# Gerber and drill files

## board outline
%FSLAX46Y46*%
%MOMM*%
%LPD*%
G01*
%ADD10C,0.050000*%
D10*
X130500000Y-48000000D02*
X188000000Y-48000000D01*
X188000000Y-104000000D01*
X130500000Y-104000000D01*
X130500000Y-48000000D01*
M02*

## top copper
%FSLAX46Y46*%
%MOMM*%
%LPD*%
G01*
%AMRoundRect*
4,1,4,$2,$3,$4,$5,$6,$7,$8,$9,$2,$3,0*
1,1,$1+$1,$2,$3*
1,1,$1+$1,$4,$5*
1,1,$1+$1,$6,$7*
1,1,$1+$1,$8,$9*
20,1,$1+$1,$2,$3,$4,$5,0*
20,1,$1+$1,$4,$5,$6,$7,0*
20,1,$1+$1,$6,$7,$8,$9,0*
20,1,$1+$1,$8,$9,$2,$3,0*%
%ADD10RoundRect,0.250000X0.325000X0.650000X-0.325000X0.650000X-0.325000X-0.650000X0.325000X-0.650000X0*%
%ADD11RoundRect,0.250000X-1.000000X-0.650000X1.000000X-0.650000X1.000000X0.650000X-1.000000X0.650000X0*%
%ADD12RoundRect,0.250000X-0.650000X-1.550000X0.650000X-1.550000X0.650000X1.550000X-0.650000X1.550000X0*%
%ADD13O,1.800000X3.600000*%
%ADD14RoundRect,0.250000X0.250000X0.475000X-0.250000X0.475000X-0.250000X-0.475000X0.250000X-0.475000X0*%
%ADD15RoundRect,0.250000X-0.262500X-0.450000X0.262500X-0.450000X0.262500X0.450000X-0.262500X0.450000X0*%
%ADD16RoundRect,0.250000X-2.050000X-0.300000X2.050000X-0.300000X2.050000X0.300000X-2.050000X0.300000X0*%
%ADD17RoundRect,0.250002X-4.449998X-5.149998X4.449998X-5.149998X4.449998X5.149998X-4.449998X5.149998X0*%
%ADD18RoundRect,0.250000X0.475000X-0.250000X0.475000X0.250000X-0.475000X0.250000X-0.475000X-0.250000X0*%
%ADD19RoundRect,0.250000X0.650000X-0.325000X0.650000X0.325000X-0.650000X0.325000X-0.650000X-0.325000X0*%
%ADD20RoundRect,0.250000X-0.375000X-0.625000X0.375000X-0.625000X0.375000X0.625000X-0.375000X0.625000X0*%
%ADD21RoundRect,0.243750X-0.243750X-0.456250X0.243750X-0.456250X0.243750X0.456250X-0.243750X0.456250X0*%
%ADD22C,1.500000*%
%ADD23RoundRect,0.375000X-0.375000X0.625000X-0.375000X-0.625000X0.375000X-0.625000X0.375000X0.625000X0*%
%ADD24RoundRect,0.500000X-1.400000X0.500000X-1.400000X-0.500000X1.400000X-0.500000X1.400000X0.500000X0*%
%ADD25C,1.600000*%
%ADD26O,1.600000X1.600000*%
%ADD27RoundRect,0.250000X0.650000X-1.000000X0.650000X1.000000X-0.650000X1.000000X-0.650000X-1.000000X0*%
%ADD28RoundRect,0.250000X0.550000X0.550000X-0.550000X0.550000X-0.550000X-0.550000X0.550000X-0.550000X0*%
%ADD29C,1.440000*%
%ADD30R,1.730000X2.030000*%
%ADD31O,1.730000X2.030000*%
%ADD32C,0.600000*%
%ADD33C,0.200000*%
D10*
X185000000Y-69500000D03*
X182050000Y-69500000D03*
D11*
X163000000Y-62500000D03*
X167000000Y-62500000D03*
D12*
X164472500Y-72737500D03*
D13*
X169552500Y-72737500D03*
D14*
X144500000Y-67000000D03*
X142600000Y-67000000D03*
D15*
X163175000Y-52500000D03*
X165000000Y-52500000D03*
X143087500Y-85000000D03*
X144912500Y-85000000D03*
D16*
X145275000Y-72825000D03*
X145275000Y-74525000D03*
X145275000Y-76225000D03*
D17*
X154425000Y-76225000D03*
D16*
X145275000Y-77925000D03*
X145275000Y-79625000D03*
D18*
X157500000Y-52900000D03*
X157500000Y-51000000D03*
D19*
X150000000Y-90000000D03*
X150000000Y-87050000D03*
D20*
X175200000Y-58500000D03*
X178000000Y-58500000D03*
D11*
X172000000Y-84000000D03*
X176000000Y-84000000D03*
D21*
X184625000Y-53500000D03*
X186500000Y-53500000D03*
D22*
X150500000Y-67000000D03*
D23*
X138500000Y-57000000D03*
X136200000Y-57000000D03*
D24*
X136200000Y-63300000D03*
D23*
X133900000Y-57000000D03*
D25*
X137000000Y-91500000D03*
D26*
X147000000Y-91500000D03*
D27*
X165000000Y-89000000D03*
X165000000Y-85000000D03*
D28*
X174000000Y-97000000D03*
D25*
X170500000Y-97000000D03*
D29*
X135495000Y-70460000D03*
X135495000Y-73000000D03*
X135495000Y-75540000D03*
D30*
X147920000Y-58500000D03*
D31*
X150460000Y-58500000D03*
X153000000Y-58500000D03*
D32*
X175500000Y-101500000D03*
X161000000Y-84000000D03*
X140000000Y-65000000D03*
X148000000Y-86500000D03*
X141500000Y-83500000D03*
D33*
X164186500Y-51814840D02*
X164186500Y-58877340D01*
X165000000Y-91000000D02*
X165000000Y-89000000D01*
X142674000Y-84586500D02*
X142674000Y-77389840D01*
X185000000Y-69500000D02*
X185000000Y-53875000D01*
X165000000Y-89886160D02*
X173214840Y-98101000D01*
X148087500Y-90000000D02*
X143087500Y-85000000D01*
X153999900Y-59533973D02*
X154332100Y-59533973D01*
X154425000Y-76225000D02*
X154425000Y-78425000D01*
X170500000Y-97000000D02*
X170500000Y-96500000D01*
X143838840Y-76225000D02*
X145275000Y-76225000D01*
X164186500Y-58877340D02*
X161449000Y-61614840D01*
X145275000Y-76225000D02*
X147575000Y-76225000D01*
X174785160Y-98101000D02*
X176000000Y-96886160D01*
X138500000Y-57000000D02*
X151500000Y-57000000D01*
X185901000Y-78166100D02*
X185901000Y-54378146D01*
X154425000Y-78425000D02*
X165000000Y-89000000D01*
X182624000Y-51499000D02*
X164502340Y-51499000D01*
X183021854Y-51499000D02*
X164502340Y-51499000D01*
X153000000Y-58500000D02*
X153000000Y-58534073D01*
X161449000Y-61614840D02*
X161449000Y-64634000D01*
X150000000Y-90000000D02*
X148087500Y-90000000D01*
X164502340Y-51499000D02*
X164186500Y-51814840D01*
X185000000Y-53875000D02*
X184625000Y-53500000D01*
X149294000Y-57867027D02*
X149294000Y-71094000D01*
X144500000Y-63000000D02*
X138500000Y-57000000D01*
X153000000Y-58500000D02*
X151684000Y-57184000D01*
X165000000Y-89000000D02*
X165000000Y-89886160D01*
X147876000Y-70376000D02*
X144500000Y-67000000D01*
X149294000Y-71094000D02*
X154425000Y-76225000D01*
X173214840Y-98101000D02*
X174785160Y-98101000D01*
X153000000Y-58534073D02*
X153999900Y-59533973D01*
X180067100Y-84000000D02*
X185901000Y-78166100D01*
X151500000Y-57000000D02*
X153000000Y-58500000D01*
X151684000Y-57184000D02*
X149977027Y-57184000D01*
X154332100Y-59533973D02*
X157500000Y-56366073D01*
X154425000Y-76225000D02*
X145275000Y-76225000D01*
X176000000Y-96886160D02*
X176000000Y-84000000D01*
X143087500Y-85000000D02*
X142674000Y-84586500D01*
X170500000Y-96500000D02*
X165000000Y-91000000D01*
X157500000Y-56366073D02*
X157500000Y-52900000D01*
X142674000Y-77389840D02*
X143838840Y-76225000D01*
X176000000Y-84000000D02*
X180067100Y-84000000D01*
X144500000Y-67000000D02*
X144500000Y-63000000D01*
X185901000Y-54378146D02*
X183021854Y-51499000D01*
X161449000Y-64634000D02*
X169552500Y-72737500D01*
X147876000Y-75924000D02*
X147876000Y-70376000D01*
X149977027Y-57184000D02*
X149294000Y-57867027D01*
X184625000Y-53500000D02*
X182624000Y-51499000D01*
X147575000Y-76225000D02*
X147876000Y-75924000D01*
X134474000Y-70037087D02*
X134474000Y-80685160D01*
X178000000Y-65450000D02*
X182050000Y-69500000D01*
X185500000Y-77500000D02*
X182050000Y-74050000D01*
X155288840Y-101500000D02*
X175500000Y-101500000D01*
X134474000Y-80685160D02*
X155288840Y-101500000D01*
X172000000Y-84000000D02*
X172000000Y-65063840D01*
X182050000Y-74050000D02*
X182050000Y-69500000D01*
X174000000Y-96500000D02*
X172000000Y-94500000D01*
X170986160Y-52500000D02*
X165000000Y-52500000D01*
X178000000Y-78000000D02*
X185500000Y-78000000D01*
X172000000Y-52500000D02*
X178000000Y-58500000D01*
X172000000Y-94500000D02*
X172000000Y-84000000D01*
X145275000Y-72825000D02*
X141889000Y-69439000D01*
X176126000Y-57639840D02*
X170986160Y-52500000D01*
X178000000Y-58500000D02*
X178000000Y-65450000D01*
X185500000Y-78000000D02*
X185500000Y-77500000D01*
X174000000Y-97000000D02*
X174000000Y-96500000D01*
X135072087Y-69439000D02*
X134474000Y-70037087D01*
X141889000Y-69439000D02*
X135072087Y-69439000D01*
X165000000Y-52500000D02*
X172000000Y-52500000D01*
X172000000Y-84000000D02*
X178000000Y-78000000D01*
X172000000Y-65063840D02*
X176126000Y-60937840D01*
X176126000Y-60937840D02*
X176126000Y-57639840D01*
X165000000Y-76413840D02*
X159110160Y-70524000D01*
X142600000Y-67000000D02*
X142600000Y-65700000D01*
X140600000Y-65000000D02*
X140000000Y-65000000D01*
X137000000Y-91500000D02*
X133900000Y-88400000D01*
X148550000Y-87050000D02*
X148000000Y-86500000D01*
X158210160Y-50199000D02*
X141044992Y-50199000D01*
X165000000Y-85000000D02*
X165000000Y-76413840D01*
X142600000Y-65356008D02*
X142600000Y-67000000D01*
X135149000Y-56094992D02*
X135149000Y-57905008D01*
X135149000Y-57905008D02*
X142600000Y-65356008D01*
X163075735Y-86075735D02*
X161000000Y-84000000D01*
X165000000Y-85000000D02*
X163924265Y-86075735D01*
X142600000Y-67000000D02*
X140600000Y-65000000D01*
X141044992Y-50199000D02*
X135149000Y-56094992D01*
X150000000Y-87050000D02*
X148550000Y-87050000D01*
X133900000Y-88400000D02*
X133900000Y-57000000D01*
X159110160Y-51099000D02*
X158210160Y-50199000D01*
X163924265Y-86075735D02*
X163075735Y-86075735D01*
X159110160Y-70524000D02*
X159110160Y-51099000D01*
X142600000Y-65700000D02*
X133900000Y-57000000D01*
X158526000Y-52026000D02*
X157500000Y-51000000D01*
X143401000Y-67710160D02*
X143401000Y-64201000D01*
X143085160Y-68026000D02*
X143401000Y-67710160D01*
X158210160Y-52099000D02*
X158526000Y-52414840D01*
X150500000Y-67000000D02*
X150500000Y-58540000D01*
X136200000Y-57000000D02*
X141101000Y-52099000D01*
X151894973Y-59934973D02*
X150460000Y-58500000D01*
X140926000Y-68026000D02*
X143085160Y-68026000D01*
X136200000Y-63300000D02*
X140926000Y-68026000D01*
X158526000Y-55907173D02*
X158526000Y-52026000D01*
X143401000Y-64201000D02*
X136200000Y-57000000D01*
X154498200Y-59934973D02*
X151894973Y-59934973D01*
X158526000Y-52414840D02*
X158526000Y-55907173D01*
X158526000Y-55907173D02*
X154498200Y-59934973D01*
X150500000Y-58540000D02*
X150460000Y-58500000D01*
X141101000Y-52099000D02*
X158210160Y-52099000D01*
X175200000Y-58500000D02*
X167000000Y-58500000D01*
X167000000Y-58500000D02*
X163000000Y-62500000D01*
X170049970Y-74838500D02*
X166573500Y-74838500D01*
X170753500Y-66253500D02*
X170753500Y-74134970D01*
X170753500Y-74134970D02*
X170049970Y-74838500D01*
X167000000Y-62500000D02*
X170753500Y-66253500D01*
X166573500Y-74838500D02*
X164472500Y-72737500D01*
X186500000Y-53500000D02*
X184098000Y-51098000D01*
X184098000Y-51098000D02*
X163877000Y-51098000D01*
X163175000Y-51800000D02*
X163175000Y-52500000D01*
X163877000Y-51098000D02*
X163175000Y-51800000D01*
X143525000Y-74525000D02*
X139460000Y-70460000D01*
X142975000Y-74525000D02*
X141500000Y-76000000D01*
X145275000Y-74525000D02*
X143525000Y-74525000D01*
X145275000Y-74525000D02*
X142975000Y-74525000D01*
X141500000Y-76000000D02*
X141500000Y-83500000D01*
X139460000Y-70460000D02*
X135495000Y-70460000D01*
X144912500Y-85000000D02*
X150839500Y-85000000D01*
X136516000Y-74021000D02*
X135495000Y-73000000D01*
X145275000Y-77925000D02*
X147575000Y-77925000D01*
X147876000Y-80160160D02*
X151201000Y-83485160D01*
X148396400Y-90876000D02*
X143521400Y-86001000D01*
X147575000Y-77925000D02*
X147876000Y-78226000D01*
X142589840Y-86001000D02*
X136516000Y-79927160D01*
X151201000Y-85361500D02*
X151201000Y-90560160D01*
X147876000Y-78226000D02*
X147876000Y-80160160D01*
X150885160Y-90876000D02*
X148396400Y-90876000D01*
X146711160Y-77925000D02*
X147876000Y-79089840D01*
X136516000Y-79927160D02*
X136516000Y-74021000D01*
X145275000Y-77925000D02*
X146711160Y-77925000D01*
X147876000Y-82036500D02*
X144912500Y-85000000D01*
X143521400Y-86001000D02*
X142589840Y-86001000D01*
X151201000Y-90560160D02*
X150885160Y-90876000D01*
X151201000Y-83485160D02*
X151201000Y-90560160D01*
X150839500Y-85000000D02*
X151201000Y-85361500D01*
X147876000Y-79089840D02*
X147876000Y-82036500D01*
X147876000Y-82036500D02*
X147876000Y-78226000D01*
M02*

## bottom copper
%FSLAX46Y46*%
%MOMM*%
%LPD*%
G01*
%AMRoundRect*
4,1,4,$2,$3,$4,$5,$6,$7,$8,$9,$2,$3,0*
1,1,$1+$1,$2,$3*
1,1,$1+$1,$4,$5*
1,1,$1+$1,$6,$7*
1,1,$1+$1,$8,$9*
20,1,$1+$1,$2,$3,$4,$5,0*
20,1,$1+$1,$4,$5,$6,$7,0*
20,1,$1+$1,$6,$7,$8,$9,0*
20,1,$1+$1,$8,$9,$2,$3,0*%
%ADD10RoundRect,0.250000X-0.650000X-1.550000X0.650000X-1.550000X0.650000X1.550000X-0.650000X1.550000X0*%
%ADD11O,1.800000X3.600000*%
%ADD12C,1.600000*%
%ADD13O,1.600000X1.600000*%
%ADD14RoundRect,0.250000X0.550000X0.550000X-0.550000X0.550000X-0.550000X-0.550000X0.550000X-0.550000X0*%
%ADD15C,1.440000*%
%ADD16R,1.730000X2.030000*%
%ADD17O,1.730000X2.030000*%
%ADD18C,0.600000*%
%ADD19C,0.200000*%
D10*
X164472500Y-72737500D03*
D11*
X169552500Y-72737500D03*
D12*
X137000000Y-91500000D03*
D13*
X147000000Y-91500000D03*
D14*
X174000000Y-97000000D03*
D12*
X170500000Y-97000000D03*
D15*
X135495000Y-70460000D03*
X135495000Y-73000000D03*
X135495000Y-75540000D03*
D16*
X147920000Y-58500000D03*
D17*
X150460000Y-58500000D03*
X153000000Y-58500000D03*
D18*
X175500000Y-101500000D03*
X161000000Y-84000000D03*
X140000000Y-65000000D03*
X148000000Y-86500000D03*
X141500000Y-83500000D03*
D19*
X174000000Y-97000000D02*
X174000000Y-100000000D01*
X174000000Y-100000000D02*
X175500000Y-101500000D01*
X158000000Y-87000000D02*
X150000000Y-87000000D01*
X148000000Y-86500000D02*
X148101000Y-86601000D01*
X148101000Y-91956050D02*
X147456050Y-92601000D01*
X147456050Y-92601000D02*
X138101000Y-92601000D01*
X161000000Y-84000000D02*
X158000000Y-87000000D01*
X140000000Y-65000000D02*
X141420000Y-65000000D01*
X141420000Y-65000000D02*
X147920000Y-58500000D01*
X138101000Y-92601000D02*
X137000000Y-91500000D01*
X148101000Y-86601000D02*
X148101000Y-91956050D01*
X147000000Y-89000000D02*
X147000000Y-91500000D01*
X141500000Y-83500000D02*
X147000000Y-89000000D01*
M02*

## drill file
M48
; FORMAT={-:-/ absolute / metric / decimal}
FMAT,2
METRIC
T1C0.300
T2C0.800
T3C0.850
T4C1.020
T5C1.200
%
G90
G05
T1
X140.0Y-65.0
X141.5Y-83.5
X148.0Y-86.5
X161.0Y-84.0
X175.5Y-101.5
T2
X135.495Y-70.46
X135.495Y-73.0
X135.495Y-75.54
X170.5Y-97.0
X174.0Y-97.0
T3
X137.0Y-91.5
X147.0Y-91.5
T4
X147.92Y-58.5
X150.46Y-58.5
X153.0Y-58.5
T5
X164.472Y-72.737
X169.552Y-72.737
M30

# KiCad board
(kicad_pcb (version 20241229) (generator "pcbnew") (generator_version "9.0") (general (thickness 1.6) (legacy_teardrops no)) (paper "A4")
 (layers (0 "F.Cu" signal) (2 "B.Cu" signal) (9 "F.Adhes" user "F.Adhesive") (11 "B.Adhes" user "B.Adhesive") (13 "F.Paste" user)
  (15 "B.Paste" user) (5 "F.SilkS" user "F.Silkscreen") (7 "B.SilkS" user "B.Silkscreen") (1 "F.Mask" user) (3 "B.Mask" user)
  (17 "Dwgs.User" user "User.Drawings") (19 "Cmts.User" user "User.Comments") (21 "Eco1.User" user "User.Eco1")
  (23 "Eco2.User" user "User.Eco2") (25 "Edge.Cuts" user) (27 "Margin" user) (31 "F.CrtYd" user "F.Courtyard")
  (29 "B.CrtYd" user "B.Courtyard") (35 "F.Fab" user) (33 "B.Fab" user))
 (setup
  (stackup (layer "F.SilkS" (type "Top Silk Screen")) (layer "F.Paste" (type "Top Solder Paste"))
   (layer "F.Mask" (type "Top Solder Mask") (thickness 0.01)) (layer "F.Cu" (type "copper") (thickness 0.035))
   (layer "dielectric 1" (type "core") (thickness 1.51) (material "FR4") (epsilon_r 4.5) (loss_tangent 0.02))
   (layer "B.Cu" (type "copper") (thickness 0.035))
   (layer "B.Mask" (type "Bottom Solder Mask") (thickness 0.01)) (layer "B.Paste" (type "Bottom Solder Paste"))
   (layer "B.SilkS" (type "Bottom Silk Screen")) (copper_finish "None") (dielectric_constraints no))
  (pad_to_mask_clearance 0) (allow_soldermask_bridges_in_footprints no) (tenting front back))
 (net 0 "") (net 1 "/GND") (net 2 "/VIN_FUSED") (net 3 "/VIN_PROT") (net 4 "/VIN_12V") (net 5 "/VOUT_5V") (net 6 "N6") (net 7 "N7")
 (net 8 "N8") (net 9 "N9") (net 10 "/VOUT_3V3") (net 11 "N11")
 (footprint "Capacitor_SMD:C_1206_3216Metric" (layer "F.Cu") (at 183.525 69.5 180)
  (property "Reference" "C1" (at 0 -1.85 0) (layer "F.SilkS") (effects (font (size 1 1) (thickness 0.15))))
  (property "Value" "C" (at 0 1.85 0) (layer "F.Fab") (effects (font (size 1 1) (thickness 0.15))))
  (pad "1" smd roundrect (at -1.475 0 180) (size 1.15 1.8) (layers "F.Cu" "F.Mask" "F.Paste") (roundrect_rratio 0.217391) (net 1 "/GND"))
  (pad "2" smd roundrect (at 1.475 0 180) (size 1.15 1.8) (layers "F.Cu" "F.Mask" "F.Paste") (roundrect_rratio 0.217391)
   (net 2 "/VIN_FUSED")))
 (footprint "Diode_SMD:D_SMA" (layer "F.Cu") (at 165 62.5)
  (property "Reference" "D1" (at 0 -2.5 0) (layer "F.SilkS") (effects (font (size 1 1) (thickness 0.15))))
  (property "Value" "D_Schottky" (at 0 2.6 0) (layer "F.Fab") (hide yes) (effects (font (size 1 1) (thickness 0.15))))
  (pad "1" smd roundrect (at -2 0) (size 2.5 1.8) (layers "F.Cu" "F.Mask" "F.Paste") (roundrect_rratio 0.1388888889) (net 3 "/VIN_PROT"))
  (pad "2" smd roundrect (at 2 0) (size 2.5 1.8) (layers "F.Cu" "F.Mask" "F.Paste") (roundrect_rratio 0.1388888889) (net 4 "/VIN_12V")))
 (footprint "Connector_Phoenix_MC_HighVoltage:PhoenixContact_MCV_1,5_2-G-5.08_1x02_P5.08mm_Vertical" (layer "F.Cu") (at 164.4725 72.7375)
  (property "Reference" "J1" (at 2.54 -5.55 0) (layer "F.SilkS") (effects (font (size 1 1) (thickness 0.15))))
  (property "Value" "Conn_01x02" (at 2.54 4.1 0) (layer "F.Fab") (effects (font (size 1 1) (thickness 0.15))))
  (pad "1" thru_hole roundrect (at 0 0) (size 1.8 3.6) (drill 1.2) (layers "*.Cu" "*.Mask") (remove_unused_layers no)
   (roundrect_rratio 0.138889) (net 4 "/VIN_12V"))
  (pad "2" thru_hole oval (at 5.08 0) (size 1.8 3.6) (drill 1.2) (layers "*.Cu" "*.Mask") (remove_unused_layers no) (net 1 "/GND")))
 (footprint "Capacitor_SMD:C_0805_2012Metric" (layer "F.Cu") (at 143.55 67 180)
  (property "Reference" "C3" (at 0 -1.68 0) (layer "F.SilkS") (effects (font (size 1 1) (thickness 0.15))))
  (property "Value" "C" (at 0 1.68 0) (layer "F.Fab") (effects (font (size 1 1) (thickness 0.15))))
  (pad "1" smd roundrect (at -0.95 0 180) (size 1 1.45) (layers "F.Cu" "F.Mask" "F.Paste") (roundrect_rratio 0.25) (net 1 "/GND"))
  (pad "2" smd roundrect (at 0.95 0 180) (size 1 1.45) (layers "F.Cu" "F.Mask" "F.Paste") (roundrect_rratio 0.25) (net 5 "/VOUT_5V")))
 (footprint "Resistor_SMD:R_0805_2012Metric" (layer "F.Cu") (at 164.0875 52.5)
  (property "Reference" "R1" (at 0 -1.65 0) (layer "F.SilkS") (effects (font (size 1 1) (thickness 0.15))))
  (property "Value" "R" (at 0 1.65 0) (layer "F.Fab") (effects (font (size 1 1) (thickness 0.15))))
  (pad "1" smd roundrect (at -0.9125 0) (size 1.025 1.4) (layers "F.Cu" "F.Mask" "F.Paste") (roundrect_rratio 0.243902) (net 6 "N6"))
  (pad "2" smd roundrect (at 0.9125 0) (size 1.025 1.4) (layers "F.Cu" "F.Mask" "F.Paste") (roundrect_rratio 0.243902) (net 2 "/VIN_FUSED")))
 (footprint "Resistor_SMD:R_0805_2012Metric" (layer "F.Cu") (at 144 85)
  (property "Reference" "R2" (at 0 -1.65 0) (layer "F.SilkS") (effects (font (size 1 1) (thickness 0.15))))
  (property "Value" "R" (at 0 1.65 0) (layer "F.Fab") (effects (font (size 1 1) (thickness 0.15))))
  (pad "1" smd roundrect (at -0.9125 0) (size 1.025 1.4) (layers "F.Cu" "F.Mask" "F.Paste") (roundrect_rratio 0.243902) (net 1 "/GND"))
  (pad "2" smd roundrect (at 0.9125 0) (size 1.025 1.4) (layers "F.Cu" "F.Mask" "F.Paste") (roundrect_rratio 0.243902) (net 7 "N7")))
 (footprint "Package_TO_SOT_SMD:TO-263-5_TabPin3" (layer "F.Cu") (at 152.925 76.225)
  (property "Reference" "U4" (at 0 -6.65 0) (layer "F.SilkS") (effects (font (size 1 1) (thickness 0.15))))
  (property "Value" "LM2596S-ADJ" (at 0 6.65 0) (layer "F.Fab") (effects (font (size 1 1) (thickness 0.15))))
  (pad "" smd roundrect (at -0.925 -2.775) (size 4.55 5.25) (layers "F.Paste") (roundrect_rratio 0.054945))
  (pad "" smd roundrect (at -0.925 2.775) (size 4.55 5.25) (layers "F.Paste") (roundrect_rratio 0.054945))
  (pad "" smd roundrect (at 3.925 -2.775) (size 4.55 5.25) (layers "F.Paste") (roundrect_rratio 0.054945))
  (pad "" smd roundrect (at 3.925 2.775) (size 4.55 5.25) (layers "F.Paste") (roundrect_rratio 0.054945))
  (pad "1" smd roundrect (at -7.65 -3.4) (size 4.6 1.1) (layers "F.Cu" "F.Mask" "F.Paste") (roundrect_rratio 0.227273) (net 2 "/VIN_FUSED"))
  (pad "2" smd roundrect (at -7.65 -1.7) (size 4.6 1.1) (layers "F.Cu" "F.Mask" "F.Paste") (roundrect_rratio 0.227273) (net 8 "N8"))
  (pad "3" smd roundrect (at -7.65 0) (size 4.6 1.1) (layers "F.Cu" "F.Mask" "F.Paste") (roundrect_rratio 0.227273) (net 1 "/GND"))
  (pad "3" smd roundrect (at 1.5 0) (size 9.4 10.8) (layers "F.Cu" "F.Mask") (roundrect_rratio 0.026596) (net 1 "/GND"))
  (pad "4" smd roundrect (at -7.65 1.7) (size 4.6 1.1) (layers "F.Cu" "F.Mask" "F.Paste") (roundrect_rratio 0.227273) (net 7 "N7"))
  (pad "5" smd roundrect (at -7.65 3.4) (size 4.6 1.1) (layers "F.Cu" "F.Mask" "F.Paste") (roundrect_rratio 0.227273) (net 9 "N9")))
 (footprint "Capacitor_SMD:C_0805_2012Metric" (layer "F.Cu") (at 157.5 51.95 90)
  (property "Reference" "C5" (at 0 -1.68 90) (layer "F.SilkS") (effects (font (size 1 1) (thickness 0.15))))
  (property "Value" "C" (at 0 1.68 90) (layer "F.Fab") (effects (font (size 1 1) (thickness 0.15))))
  (pad "1" smd roundrect (at -0.95 0 90) (size 1 1.45) (layers "F.Cu" "F.Mask" "F.Paste") (roundrect_rratio 0.25) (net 1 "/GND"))
  (pad "2" smd roundrect (at 0.95 0 90) (size 1 1.45) (layers "F.Cu" "F.Mask" "F.Paste") (roundrect_rratio 0.25) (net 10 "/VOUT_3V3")))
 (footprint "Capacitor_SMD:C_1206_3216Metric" (layer "F.Cu") (at 150 88.525 90)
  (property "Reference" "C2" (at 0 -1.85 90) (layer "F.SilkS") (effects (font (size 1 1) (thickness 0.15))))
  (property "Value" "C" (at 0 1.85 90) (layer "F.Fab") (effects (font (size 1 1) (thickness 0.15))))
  (pad "1" smd roundrect (at -1.475 0 90) (size 1.15 1.8) (layers "F.Cu" "F.Mask" "F.Paste") (roundrect_rratio 0.217391) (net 1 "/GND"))
  (pad "2" smd roundrect (at 1.475 0 90) (size 1.15 1.8) (layers "F.Cu" "F.Mask" "F.Paste") (roundrect_rratio 0.217391) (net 5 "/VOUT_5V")))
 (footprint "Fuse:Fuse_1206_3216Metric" (layer "F.Cu") (at 176.6 58.5)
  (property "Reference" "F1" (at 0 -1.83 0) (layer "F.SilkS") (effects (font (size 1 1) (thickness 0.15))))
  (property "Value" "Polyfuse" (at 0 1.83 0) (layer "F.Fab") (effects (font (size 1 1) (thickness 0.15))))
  (pad "1" smd roundrect (at -1.4 0) (size 1.25 1.75) (layers "F.Cu" "F.Mask" "F.Paste") (roundrect_rratio 0.2) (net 3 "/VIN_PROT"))
  (pad "2" smd roundrect (at 1.4 0) (size 1.25 1.75) (layers "F.Cu" "F.Mask" "F.Paste") (roundrect_rratio 0.2) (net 2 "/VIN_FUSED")))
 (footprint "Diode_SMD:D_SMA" (layer "F.Cu") (at 174 84)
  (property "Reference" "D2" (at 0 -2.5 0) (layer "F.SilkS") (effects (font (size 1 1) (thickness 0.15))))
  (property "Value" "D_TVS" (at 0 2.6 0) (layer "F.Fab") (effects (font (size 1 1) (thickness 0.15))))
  (pad "1" smd roundrect (at -2 0) (size 2.5 1.8) (layers "F.Cu" "F.Mask" "F.Paste") (roundrect_rratio 0.1388888889) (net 2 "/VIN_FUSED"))
  (pad "2" smd roundrect (at 2 0) (size 2.5 1.8) (layers "F.Cu" "F.Mask" "F.Paste") (roundrect_rratio 0.1388888889) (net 1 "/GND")))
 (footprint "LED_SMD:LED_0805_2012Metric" (layer "F.Cu") (at 185.5625 53.5)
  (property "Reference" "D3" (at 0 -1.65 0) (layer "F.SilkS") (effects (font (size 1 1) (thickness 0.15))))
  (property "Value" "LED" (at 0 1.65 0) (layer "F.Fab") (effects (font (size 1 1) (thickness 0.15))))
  (pad "1" smd roundrect (at -0.9375 0) (size 0.975 1.4) (layers "F.Cu" "F.Mask" "F.Paste") (roundrect_rratio 0.25) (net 1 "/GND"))
  (pad "2" smd roundrect (at 0.9375 0) (size 0.975 1.4) (layers "F.Cu" "F.Mask" "F.Paste") (roundrect_rratio 0.25) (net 6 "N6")))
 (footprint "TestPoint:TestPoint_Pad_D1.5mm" (layer "F.Cu") (at 150.5 67)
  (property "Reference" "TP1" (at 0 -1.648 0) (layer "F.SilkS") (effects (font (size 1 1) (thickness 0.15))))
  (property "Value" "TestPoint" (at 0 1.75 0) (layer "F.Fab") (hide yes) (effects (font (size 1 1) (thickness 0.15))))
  (pad "1" smd circle (at 0 0) (size 1.5 1.5) (layers "F.Cu" "F.Mask") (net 10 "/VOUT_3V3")))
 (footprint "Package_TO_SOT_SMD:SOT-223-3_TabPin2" (layer "F.Cu") (at 136.2 60.15 -90)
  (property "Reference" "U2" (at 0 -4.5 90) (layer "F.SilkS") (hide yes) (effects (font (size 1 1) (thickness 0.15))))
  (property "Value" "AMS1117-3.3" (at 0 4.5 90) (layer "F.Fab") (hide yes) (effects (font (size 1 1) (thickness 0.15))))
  (pad "1" smd roundrect (at -3.15 -2.3 270) (size 2 1.5) (layers "F.Cu" "F.Mask" "F.Paste") (roundrect_rratio 0.25) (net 1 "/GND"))
  (pad "2" smd roundrect (at -3.15 0 270) (size 2 1.5) (layers "F.Cu" "F.Mask" "F.Paste") (roundrect_rratio 0.25) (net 10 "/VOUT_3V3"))
  (pad "2" smd roundrect (at 3.15 0 270) (size 2 3.8) (layers "F.Cu" "F.Mask" "F.Paste") (roundrect_rratio 0.25) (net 10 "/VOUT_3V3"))
  (pad "3" smd roundrect (at -3.15 2.3 270) (size 2 1.5) (layers "F.Cu" "F.Mask" "F.Paste") (roundrect_rratio 0.25) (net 5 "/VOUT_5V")))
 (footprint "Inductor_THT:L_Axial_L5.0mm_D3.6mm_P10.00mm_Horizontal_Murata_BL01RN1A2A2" (layer "F.Cu") (at 137 91.5)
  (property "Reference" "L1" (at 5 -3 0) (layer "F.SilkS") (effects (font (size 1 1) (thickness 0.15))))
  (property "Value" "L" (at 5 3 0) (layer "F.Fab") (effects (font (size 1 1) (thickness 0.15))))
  (pad "1" thru_hole circle (at 0 0) (size 1.6 1.6) (drill 0.85) (layers "*.Cu" "*.Mask") (remove_unused_layers no) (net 5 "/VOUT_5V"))
  (pad "2" thru_hole oval (at 10 0) (size 1.6 1.6) (drill 0.85) (layers "*.Cu" "*.Mask") (remove_unused_layers no) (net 8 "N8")))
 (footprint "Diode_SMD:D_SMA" (layer "F.Cu") (at 165 87 90)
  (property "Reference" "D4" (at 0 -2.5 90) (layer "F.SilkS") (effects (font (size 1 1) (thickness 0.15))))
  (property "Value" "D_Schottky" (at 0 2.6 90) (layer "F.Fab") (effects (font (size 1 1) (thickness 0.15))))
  (pad "1" smd roundrect (at -2 0 90) (size 2.5 1.8) (layers "F.Cu" "F.Mask" "F.Paste") (roundrect_rratio 0.1388888889) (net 1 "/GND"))
  (pad "2" smd roundrect (at 2 0 90) (size 2.5 1.8) (layers "F.Cu" "F.Mask" "F.Paste") (roundrect_rratio 0.1388888889) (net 5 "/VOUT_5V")))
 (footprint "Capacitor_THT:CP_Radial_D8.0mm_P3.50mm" (layer "F.Cu") (at 174 97 180)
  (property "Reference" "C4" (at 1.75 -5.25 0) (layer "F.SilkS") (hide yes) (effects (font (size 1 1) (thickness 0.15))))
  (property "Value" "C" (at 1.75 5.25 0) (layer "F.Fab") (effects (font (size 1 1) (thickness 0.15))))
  (pad "1" thru_hole roundrect (at 0 0 180) (size 1.6 1.6) (drill 0.8) (layers "*.Cu" "*.Mask") (remove_unused_layers no)
   (roundrect_rratio 0.15625) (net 2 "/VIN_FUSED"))
  (pad "2" thru_hole circle (at 3.5 0 180) (size 1.6 1.6) (drill 0.8) (layers "*.Cu" "*.Mask") (remove_unused_layers no) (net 1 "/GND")))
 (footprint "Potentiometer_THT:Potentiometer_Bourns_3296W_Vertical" (layer "F.Cu") (at 135.495 70.46 90)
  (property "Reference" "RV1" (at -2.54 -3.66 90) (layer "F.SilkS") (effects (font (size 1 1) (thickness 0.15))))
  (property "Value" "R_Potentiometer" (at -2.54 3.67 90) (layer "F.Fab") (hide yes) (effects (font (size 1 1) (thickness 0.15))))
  (pad "1" thru_hole circle (at 0 0 90) (size 1.44 1.44) (drill 0.8) (layers "*.Cu" "*.Mask") (remove_unused_layers no) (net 8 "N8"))
  (pad "2" thru_hole circle (at -2.54 0 90) (size 1.44 1.44) (drill 0.8) (layers "*.Cu" "*.Mask") (remove_unused_layers no) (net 7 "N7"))
  (pad "3" thru_hole circle (at -5.08 0 90) (size 1.44 1.44) (drill 0.8) (layers "*.Cu" "*.Mask") (remove_unused_layers no) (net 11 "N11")))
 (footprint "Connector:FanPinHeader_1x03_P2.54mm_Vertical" (layer "F.Cu") (at 147.92 58.5)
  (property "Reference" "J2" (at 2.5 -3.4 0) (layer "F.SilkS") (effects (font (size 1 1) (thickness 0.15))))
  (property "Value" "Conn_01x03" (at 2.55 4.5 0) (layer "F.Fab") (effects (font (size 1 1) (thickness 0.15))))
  (pad "1" thru_hole rect (at 0 0 90) (size 2.03 1.73) (drill 1.02) (layers "*.Cu" "*.Mask") (remove_unused_layers no) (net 5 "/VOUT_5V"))
  (pad "2" thru_hole oval (at 2.54 0 90) (size 2.03 1.73) (drill 1.02) (layers "*.Cu" "*.Mask") (remove_unused_layers no)
   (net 10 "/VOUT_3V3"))
  (pad "3" thru_hole oval (at 5.08 0 90) (size 2.03 1.73) (drill 1.02) (layers "*.Cu" "*.Mask") (remove_unused_layers no) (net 1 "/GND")))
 (gr_rect (start 130.5 48) (end 188 104) (stroke (width 0.05) (type default)) (fill no) (layer "Edge.Cuts"))
 (segment (start 164.1865 51.81484) (end 164.1865 58.87734) (width 0.2) (layer "F.Cu") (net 1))
 (segment (start 165 91) (end 165 89) (width 0.2) (layer "F.Cu") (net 1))
 (segment (start 142.674 84.5865) (end 142.674 77.38984) (width 0.2) (layer "F.Cu") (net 1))
 (segment (start 185 69.5) (end 185 53.875) (width 0.2) (layer "F.Cu") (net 1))
 (segment (start 165 89.88616) (end 173.21484 98.101) (width 0.2) (layer "F.Cu") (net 1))
 (segment (start 148.0875 90) (end 143.0875 85) (width 0.2) (layer "F.Cu") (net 1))
 (segment (start 153.9999 59.533973) (end 154.3321 59.533973) (width 0.2) (layer "F.Cu") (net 1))
 (segment (start 154.425 76.225) (end 154.425 78.425) (width 0.2) (layer "F.Cu") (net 1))
 (segment (start 170.5 97) (end 170.5 96.5) (width 0.2) (layer "F.Cu") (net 1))
 (segment (start 143.83884 76.225) (end 145.275 76.225) (width 0.2) (layer "F.Cu") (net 1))
 (segment (start 164.1865 58.87734) (end 161.449 61.61484) (width 0.2) (layer "F.Cu") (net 1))
 (segment (start 145.275 76.225) (end 147.575 76.225) (width 0.2) (layer "F.Cu") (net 1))
 (segment (start 174.78516 98.101) (end 176 96.88616) (width 0.2) (layer "F.Cu") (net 1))
 (segment (start 138.5 57) (end 151.5 57) (width 0.2) (layer "F.Cu") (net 1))
 (segment (start 185.901 78.1661) (end 185.901 54.378146) (width 0.2) (layer "F.Cu") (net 1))
 (segment (start 154.425 78.425) (end 165 89) (width 0.2) (layer "F.Cu") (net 1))
 (segment (start 182.624 51.499) (end 164.50234 51.499) (width 0.2) (layer "F.Cu") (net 1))
 (segment (start 183.021854 51.499) (end 164.50234 51.499) (width 0.2) (layer "F.Cu") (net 1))
 (segment (start 153 58.5) (end 153 58.534073) (width 0.2) (layer "F.Cu") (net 1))
 (segment (start 161.449 61.61484) (end 161.449 64.634) (width 0.2) (layer "F.Cu") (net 1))
 (segment (start 150 90) (end 148.0875 90) (width 0.2) (layer "F.Cu") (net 1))
 (segment (start 164.50234 51.499) (end 164.1865 51.81484) (width 0.2) (layer "F.Cu") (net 1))
 (segment (start 185 53.875) (end 184.625 53.5) (width 0.2) (layer "F.Cu") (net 1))
 (segment (start 149.294 57.867027) (end 149.294 71.094) (width 0.2) (layer "F.Cu") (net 1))
 (segment (start 144.5 63) (end 138.5 57) (width 0.2) (layer "F.Cu") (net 1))
 (segment (start 153 58.5) (end 151.684 57.184) (width 0.2) (layer "F.Cu") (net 1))
 (segment (start 165 89) (end 165 89.88616) (width 0.2) (layer "F.Cu") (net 1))
 (segment (start 147.876 70.376) (end 144.5 67) (width 0.2) (layer "F.Cu") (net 1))
 (segment (start 149.294 71.094) (end 154.425 76.225) (width 0.2) (layer "F.Cu") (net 1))
 (segment (start 173.21484 98.101) (end 174.78516 98.101) (width 0.2) (layer "F.Cu") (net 1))
 (segment (start 153 58.534073) (end 153.9999 59.533973) (width 0.2) (layer "F.Cu") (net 1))
 (segment (start 180.0671 84) (end 185.901 78.1661) (width 0.2) (layer "F.Cu") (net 1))
 (segment (start 151.5 57) (end 153 58.5) (width 0.2) (layer "F.Cu") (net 1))
 (segment (start 151.684 57.184) (end 149.977027 57.184) (width 0.2) (layer "F.Cu") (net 1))
 (segment (start 154.3321 59.533973) (end 157.5 56.366073) (width 0.2) (layer "F.Cu") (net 1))
 (segment (start 154.425 76.225) (end 145.275 76.225) (width 0.2) (layer "F.Cu") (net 1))
 (segment (start 176 96.88616) (end 176 84) (width 0.2) (layer "F.Cu") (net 1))
 (segment (start 143.0875 85) (end 142.674 84.5865) (width 0.2) (layer "F.Cu") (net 1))
 (segment (start 170.5 96.5) (end 165 91) (width 0.2) (layer "F.Cu") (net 1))
 (segment (start 157.5 56.366073) (end 157.5 52.9) (width 0.2) (layer "F.Cu") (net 1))
 (segment (start 142.674 77.38984) (end 143.83884 76.225) (width 0.2) (layer "F.Cu") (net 1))
 (segment (start 176 84) (end 180.0671 84) (width 0.2) (layer "F.Cu") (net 1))
 (segment (start 144.5 67) (end 144.5 63) (width 0.2) (layer "F.Cu") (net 1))
 (segment (start 185.901 54.378146) (end 183.021854 51.499) (width 0.2) (layer "F.Cu") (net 1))
 (segment (start 161.449 64.634) (end 169.5525 72.7375) (width 0.2) (layer "F.Cu") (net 1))
 (segment (start 147.876 75.924) (end 147.876 70.376) (width 0.2) (layer "F.Cu") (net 1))
 (segment (start 149.977027 57.184) (end 149.294 57.867027) (width 0.2) (layer "F.Cu") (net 1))
 (segment (start 184.625 53.5) (end 182.624 51.499) (width 0.2) (layer "F.Cu") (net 1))
 (segment (start 147.575 76.225) (end 147.876 75.924) (width 0.2) (layer "F.Cu") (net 1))
 (segment (start 134.474 70.037087) (end 134.474 80.68516) (width 0.2) (layer "F.Cu") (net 2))
 (segment (start 178 65.45) (end 182.05 69.5) (width 0.2) (layer "F.Cu") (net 2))
 (segment (start 185.5 77.5) (end 182.05 74.05) (width 0.2) (layer "F.Cu") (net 2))
 (segment (start 155.28884 101.5) (end 175.5 101.5) (width 0.2) (layer "F.Cu") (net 2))
 (segment (start 134.474 80.68516) (end 155.28884 101.5) (width 0.2) (layer "F.Cu") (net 2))
 (segment (start 172 84) (end 172 65.06384) (width 0.2) (layer "F.Cu") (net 2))
 (segment (start 182.05 74.05) (end 182.05 69.5) (width 0.2) (layer "F.Cu") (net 2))
 (segment (start 174 96.5) (end 172 94.5) (width 0.2) (layer "F.Cu") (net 2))
 (segment (start 170.98616 52.5) (end 165 52.5) (width 0.2) (layer "F.Cu") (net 2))
 (segment (start 178 78) (end 185.5 78) (width 0.2) (layer "F.Cu") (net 2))
 (segment (start 172 52.5) (end 178 58.5) (width 0.2) (layer "F.Cu") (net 2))
 (segment (start 172 94.5) (end 172 84) (width 0.2) (layer "F.Cu") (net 2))
 (segment (start 145.275 72.825) (end 141.889 69.439) (width 0.2) (layer "F.Cu") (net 2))
 (segment (start 176.126 57.63984) (end 170.98616 52.5) (width 0.2) (layer "F.Cu") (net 2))
 (segment (start 178 58.5) (end 178 65.45) (width 0.2) (layer "F.Cu") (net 2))
 (segment (start 185.5 78) (end 185.5 77.5) (width 0.2) (layer "F.Cu") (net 2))
 (segment (start 174 97) (end 174 96.5) (width 0.2) (layer "F.Cu") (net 2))
 (segment (start 135.072087 69.439) (end 134.474 70.037087) (width 0.2) (layer "F.Cu") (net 2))
 (segment (start 141.889 69.439) (end 135.072087 69.439) (width 0.2) (layer "F.Cu") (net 2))
 (segment (start 165 52.5) (end 172 52.5) (width 0.2) (layer "F.Cu") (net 2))
 (segment (start 172 84) (end 178 78) (width 0.2) (layer "F.Cu") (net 2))
 (segment (start 172 65.06384) (end 176.126 60.93784) (width 0.2) (layer "F.Cu") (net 2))
 (segment (start 176.126 60.93784) (end 176.126 57.63984) (width 0.2) (layer "F.Cu") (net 2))
 (via (at 175.5 101.5) (size 0.6) (drill 0.3) (layers "F.Cu" "B.Cu") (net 2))
 (segment (start 174 97) (end 174 100) (width 0.2) (layer "B.Cu") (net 2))
 (segment (start 174 100) (end 175.5 101.5) (width 0.2) (layer "B.Cu") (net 2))
 (segment (start 165 76.41384) (end 159.11016 70.524) (width 0.2) (layer "F.Cu") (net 5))
 (segment (start 142.6 67) (end 142.6 65.7) (width 0.2) (layer "F.Cu") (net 5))
 (segment (start 140.6 65) (end 140 65) (width 0.2) (layer "F.Cu") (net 5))
 (segment (start 137 91.5) (end 133.9 88.4) (width 0.2) (layer "F.Cu") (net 5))
 (segment (start 148.55 87.05) (end 148 86.5) (width 0.2) (layer "F.Cu") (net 5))
 (segment (start 158.21016 50.199) (end 141.044992 50.199) (width 0.2) (layer "F.Cu") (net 5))
 (segment (start 165 85) (end 165 76.41384) (width 0.2) (layer "F.Cu") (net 5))
 (segment (start 142.6 65.356008) (end 142.6 67) (width 0.2) (layer "F.Cu") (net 5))
 (segment (start 135.149 56.094992) (end 135.149 57.905008) (width 0.2) (layer "F.Cu") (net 5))
 (segment (start 135.149 57.905008) (end 142.6 65.356008) (width 0.2) (layer "F.Cu") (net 5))
 (segment (start 163.075735 86.075735) (end 161 84) (width 0.2) (layer "F.Cu") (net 5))
 (segment (start 165 85) (end 163.924265 86.075735) (width 0.2) (layer "F.Cu") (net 5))
 (segment (start 142.6 67) (end 140.6 65) (width 0.2) (layer "F.Cu") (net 5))
 (segment (start 141.044992 50.199) (end 135.149 56.094992) (width 0.2) (layer "F.Cu") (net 5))
 (segment (start 150 87.05) (end 148.55 87.05) (width 0.2) (layer "F.Cu") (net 5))
 (segment (start 133.9 88.4) (end 133.9 57) (width 0.2) (layer "F.Cu") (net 5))
 (segment (start 159.11016 51.099) (end 158.21016 50.199) (width 0.2) (layer "F.Cu") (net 5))
 (segment (start 163.924265 86.075735) (end 163.075735 86.075735) (width 0.2) (layer "F.Cu") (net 5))
 (segment (start 159.11016 70.524) (end 159.11016 51.099) (width 0.2) (layer "F.Cu") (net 5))
 (segment (start 142.6 65.7) (end 133.9 57) (width 0.2) (layer "F.Cu") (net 5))
 (via (at 161 84) (size 0.6) (drill 0.3) (layers "F.Cu" "B.Cu") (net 5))
 (via (at 140 65) (size 0.6) (drill 0.3) (layers "F.Cu" "B.Cu") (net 5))
 (via (at 148 86.5) (size 0.6) (drill 0.3) (layers "F.Cu" "B.Cu") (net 5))
 (segment (start 158 87) (end 150 87) (width 0.2) (layer "B.Cu") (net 5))
 (segment (start 148 86.5) (end 148.101 86.601) (width 0.2) (layer "B.Cu") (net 5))
 (segment (start 148.101 91.95605) (end 147.45605 92.601) (width 0.2) (layer "B.Cu") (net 5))
 (segment (start 147.45605 92.601) (end 138.101 92.601) (width 0.2) (layer "B.Cu") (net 5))
 (segment (start 161 84) (end 158 87) (width 0.2) (layer "B.Cu") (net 5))
 (segment (start 140 65) (end 141.42 65) (width 0.2) (layer "B.Cu") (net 5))
 (segment (start 141.42 65) (end 147.92 58.5) (width 0.2) (layer "B.Cu") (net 5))
 (segment (start 138.101 92.601) (end 137 91.5) (width 0.2) (layer "B.Cu") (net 5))
 (segment (start 148.101 86.601) (end 148.101 91.95605) (width 0.2) (layer "B.Cu") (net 5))
 (segment (start 158.526 52.026) (end 157.5 51) (width 0.2) (layer "F.Cu") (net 10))
 (segment (start 143.401 67.71016) (end 143.401 64.201) (width 0.2) (layer "F.Cu") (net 10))
 (segment (start 143.08516 68.026) (end 143.401 67.71016) (width 0.2) (layer "F.Cu") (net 10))
 (segment (start 158.21016 52.099) (end 158.526 52.41484) (width 0.2) (layer "F.Cu") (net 10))
 (segment (start 150.5 67) (end 150.5 58.54) (width 0.2) (layer "F.Cu") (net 10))
 (segment (start 136.2 57) (end 141.101 52.099) (width 0.2) (layer "F.Cu") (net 10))
 (segment (start 151.894973 59.934973) (end 150.46 58.5) (width 0.2) (layer "F.Cu") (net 10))
 (segment (start 140.926 68.026) (end 143.08516 68.026) (width 0.2) (layer "F.Cu") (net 10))
 (segment (start 136.2 63.3) (end 140.926 68.026) (width 0.2) (layer "F.Cu") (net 10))
 (segment (start 158.526 55.907173) (end 158.526 52.026) (width 0.2) (layer "F.Cu") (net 10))
 (segment (start 143.401 64.201) (end 136.2 57) (width 0.2) (layer "F.Cu") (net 10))
 (segment (start 154.4982 59.934973) (end 151.894973 59.934973) (width 0.2) (layer "F.Cu") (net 10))
 (segment (start 158.526 52.41484) (end 158.526 55.907173) (width 0.2) (layer "F.Cu") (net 10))
 (segment (start 158.526 55.907173) (end 154.4982 59.934973) (width 0.2) (layer "F.Cu") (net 10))
 (segment (start 150.5 58.54) (end 150.46 58.5) (width 0.2) (layer "F.Cu") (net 10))
 (segment (start 141.101 52.099) (end 158.21016 52.099) (width 0.2) (layer "F.Cu") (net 10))
 (segment (start 175.2 58.5) (end 167 58.5) (width 0.2) (layer "F.Cu") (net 3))
 (segment (start 167 58.5) (end 163 62.5) (width 0.2) (layer "F.Cu") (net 3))
 (segment (start 170.04997 74.8385) (end 166.5735 74.8385) (width 0.2) (layer "F.Cu") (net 4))
 (segment (start 170.7535 66.2535) (end 170.7535 74.13497) (width 0.2) (layer "F.Cu") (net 4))
 (segment (start 170.7535 74.13497) (end 170.04997 74.8385) (width 0.2) (layer "F.Cu") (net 4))
 (segment (start 167 62.5) (end 170.7535 66.2535) (width 0.2) (layer "F.Cu") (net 4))
 (segment (start 166.5735 74.8385) (end 164.4725 72.7375) (width 0.2) (layer "F.Cu") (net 4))
 (segment (start 186.5 53.5) (end 184.098 51.098) (width 0.2) (layer "F.Cu") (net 6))
 (segment (start 184.098 51.098) (end 163.877 51.098) (width 0.2) (layer "F.Cu") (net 6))
 (segment (start 163.175 51.8) (end 163.175 52.5) (width 0.2) (layer "F.Cu") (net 6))
 (segment (start 163.877 51.098) (end 163.175 51.8) (width 0.2) (layer "F.Cu") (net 6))
 (segment (start 143.525 74.525) (end 139.46 70.46) (width 0.2) (layer "F.Cu") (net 8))
 (segment (start 142.975 74.525) (end 141.5 76) (width 0.2) (layer "F.Cu") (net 8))
 (segment (start 145.275 74.525) (end 143.525 74.525) (width 0.2) (layer "F.Cu") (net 8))
 (segment (start 145.275 74.525) (end 142.975 74.525) (width 0.2) (layer "F.Cu") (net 8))
 (segment (start 141.5 76) (end 141.5 83.5) (width 0.2) (layer "F.Cu") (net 8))
 (segment (start 139.46 70.46) (end 135.495 70.46) (width 0.2) (layer "F.Cu") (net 8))
 (via (at 141.5 83.5) (size 0.6) (drill 0.3) (layers "F.Cu" "B.Cu") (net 8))
 (segment (start 147 89) (end 147 91.5) (width 0.2) (layer "B.Cu") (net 8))
 (segment (start 141.5 83.5) (end 147 89) (width 0.2) (layer "B.Cu") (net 8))
 (segment (start 144.9125 85) (end 150.8395 85) (width 0.2) (layer "F.Cu") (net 7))
 (segment (start 136.516 74.021) (end 135.495 73) (width 0.2) (layer "F.Cu") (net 7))
 (segment (start 145.275 77.925) (end 147.575 77.925) (width 0.2) (layer "F.Cu") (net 7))
 (segment (start 147.876 80.16016) (end 151.201 83.48516) (width 0.2) (layer "F.Cu") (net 7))
 (segment (start 148.3964 90.876) (end 143.5214 86.001) (width 0.2) (layer "F.Cu") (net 7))
 (segment (start 147.575 77.925) (end 147.876 78.226) (width 0.2) (layer "F.Cu") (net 7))
 (segment (start 142.58984 86.001) (end 136.516 79.92716) (width 0.2) (layer "F.Cu") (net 7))
 (segment (start 151.201 85.3615) (end 151.201 90.56016) (width 0.2) (layer "F.Cu") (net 7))
 (segment (start 147.876 78.226) (end 147.876 80.16016) (width 0.2) (layer "F.Cu") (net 7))
 (segment (start 150.88516 90.876) (end 148.3964 90.876) (width 0.2) (layer "F.Cu") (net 7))
 (segment (start 146.71116 77.925) (end 147.876 79.08984) (width 0.2) (layer "F.Cu") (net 7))
 (segment (start 136.516 79.92716) (end 136.516 74.021) (width 0.2) (layer "F.Cu") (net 7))
 (segment (start 145.275 77.925) (end 146.71116 77.925) (width 0.2) (layer "F.Cu") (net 7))
 (segment (start 147.876 82.0365) (end 144.9125 85) (width 0.2) (layer "F.Cu") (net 7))
 (segment (start 143.5214 86.001) (end 142.58984 86.001) (width 0.2) (layer "F.Cu") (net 7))
 (segment (start 151.201 90.56016) (end 150.88516 90.876) (width 0.2) (layer "F.Cu") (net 7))
 (segment (start 151.201 83.48516) (end 151.201 90.56016) (width 0.2) (layer "F.Cu") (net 7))
 (segment (start 150.8395 85) (end 151.201 85.3615) (width 0.2) (layer "F.Cu") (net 7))
 (segment (start 147.876 79.08984) (end 147.876 82.0365) (width 0.2) (layer "F.Cu") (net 7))
 (segment (start 147.876 82.0365) (end 147.876 78.226) (width 0.2) (layer "F.Cu") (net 7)))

